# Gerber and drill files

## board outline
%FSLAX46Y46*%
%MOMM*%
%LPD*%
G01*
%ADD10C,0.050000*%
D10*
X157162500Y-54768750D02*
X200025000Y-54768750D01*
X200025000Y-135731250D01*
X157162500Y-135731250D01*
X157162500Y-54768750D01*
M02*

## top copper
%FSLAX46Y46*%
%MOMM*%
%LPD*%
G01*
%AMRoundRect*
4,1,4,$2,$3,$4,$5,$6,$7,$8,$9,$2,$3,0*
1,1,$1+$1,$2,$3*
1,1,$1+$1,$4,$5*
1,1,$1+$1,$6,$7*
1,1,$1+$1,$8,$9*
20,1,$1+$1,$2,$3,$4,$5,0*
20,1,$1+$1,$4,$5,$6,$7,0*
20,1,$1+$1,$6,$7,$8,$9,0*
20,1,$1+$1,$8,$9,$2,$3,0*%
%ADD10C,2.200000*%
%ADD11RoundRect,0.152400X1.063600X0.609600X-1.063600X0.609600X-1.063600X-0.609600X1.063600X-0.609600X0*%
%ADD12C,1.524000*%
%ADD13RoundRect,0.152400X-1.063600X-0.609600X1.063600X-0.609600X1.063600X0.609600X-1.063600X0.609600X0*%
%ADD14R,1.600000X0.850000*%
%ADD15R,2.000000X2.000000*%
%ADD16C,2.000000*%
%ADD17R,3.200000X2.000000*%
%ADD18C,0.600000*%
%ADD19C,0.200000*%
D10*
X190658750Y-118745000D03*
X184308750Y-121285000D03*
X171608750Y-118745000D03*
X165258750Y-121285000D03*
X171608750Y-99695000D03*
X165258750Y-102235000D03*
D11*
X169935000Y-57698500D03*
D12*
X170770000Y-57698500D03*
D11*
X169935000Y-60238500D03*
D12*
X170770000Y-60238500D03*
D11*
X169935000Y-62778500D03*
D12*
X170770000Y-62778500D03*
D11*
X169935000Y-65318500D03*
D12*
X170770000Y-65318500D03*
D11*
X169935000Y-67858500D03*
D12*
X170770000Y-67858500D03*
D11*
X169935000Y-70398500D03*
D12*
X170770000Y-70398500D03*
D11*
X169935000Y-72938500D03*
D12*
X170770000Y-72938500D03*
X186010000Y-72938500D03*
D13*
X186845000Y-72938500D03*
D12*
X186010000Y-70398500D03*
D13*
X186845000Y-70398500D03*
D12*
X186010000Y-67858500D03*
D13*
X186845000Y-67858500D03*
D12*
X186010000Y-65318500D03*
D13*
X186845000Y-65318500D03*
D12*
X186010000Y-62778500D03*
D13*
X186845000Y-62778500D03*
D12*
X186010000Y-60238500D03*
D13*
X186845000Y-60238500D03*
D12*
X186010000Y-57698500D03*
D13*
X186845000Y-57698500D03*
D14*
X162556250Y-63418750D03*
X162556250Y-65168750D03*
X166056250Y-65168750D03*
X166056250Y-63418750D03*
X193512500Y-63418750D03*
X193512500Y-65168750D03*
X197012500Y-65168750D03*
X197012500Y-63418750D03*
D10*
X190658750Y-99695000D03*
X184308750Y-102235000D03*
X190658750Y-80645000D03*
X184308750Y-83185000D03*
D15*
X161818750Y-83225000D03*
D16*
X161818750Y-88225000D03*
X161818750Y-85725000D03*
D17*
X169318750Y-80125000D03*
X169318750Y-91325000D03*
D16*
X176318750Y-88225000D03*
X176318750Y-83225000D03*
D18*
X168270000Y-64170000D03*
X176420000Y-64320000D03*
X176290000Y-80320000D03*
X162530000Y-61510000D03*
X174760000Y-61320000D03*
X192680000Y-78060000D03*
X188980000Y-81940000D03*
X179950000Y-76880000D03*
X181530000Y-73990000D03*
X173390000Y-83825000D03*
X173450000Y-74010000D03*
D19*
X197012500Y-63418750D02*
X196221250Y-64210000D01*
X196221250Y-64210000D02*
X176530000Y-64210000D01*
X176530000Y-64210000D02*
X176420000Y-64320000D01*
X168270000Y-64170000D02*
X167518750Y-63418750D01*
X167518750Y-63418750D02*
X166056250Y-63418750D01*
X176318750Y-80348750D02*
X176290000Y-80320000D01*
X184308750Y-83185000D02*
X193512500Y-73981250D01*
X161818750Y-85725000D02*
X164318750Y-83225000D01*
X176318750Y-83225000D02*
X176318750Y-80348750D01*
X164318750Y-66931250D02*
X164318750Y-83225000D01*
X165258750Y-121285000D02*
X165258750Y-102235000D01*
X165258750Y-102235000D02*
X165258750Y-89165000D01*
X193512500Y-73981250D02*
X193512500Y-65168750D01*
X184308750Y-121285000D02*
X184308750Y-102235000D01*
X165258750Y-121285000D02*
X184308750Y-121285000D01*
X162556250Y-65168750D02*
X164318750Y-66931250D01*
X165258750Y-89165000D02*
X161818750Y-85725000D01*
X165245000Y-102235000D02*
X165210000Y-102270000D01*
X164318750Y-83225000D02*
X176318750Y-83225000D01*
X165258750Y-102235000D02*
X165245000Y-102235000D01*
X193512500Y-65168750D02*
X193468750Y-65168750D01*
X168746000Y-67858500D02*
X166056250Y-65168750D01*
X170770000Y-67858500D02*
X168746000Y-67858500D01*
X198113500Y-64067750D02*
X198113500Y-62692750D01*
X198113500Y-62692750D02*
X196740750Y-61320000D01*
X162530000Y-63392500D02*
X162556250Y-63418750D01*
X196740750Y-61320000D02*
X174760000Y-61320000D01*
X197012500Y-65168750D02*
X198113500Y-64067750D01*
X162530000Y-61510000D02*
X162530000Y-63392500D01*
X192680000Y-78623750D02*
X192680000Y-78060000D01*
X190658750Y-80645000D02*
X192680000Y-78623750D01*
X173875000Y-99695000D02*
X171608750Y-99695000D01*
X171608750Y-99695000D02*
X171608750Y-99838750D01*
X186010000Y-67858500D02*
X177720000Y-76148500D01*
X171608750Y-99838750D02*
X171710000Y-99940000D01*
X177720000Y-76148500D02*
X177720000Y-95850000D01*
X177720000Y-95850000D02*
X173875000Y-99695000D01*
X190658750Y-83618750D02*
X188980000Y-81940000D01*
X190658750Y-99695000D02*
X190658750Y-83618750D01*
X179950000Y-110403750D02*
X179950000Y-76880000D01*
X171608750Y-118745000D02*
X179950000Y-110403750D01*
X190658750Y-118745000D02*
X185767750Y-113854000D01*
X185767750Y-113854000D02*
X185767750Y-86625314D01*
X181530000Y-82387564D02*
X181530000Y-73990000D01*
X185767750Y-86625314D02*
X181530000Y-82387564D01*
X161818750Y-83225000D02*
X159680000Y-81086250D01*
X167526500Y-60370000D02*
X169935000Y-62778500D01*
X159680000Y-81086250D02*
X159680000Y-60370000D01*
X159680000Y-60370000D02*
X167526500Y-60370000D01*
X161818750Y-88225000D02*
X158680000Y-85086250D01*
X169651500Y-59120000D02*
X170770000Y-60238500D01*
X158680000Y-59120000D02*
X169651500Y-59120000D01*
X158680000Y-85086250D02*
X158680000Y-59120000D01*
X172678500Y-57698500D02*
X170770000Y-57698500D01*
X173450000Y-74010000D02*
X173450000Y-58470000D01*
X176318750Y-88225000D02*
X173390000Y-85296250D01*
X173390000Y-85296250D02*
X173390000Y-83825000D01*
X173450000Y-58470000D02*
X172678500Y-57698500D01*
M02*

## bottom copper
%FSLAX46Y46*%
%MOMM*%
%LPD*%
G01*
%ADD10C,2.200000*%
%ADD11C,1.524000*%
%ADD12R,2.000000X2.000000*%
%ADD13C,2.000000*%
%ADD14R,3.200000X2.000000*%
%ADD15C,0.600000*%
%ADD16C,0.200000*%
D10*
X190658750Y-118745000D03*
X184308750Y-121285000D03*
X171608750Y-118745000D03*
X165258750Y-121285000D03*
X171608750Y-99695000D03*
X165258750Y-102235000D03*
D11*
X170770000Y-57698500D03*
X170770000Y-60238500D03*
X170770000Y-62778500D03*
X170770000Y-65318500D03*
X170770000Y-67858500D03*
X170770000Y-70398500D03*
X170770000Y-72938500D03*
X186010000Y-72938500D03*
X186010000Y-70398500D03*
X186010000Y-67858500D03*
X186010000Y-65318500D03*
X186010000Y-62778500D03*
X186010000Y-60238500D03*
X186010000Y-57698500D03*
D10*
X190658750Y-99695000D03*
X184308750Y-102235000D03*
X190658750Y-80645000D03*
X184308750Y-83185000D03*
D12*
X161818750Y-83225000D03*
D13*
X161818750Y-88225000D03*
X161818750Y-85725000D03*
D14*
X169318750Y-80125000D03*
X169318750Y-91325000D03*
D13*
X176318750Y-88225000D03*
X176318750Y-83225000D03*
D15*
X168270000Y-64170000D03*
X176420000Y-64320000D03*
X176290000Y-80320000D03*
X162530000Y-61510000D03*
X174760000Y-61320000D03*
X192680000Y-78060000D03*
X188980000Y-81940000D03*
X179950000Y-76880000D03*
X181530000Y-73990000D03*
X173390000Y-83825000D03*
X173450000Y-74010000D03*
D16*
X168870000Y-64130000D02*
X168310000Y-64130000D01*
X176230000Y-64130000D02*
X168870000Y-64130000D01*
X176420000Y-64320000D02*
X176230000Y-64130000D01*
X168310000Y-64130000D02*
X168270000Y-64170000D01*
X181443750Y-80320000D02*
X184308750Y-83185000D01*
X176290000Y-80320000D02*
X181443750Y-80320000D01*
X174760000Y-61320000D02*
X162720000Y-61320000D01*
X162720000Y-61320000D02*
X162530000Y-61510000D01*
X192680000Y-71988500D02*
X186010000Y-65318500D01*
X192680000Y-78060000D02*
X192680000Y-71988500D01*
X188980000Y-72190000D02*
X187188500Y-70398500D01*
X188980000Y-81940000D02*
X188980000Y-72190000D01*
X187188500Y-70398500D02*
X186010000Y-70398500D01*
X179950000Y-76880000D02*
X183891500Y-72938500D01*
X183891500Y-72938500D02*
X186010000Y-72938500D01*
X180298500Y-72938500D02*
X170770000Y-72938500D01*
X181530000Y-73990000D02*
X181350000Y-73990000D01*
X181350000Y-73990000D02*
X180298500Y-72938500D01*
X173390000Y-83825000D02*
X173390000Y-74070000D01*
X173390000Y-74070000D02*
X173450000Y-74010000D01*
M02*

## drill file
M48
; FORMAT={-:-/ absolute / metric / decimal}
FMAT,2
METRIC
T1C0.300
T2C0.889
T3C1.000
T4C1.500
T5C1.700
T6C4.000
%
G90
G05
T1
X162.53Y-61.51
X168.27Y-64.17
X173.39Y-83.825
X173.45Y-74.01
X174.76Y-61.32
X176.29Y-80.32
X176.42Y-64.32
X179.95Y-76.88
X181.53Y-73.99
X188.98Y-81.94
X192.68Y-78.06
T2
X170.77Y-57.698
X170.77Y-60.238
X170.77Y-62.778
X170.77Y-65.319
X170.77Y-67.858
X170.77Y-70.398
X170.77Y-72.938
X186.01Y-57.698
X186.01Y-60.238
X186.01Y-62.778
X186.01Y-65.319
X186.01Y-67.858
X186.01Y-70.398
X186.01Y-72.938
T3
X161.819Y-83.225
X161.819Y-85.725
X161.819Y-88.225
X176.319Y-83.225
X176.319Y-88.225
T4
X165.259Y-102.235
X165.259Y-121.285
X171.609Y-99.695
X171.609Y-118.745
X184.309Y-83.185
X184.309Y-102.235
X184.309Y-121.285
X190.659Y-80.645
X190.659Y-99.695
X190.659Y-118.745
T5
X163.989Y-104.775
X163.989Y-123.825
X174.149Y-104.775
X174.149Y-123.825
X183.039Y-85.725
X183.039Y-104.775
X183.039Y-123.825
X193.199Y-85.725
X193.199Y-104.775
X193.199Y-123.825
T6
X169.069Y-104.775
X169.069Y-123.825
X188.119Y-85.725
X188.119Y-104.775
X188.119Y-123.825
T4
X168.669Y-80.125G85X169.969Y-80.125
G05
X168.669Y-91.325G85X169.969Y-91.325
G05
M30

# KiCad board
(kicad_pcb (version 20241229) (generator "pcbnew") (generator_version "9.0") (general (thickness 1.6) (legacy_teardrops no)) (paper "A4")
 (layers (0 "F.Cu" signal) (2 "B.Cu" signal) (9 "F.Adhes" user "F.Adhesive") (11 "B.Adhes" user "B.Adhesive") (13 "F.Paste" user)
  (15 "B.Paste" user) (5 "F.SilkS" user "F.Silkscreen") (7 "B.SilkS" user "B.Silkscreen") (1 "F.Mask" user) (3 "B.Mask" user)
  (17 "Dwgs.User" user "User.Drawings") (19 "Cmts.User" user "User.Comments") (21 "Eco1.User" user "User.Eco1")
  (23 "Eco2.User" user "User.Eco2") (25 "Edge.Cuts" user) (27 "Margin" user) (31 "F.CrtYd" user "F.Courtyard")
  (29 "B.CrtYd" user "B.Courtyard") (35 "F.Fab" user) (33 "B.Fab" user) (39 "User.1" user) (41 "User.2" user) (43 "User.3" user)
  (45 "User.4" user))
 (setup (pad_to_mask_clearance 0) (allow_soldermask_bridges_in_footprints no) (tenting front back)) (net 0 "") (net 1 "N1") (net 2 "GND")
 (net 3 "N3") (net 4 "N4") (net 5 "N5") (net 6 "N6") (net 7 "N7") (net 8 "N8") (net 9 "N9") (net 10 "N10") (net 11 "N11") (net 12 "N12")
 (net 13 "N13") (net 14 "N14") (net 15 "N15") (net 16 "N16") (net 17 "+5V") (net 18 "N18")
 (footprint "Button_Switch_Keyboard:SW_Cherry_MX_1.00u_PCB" (layer "F.Cu") (at 190.65875 118.745)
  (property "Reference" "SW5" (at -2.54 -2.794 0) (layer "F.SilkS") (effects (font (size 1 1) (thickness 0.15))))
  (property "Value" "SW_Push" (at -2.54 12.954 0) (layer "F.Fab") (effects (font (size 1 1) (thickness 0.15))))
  (pad "" np_thru_hole circle (at -7.62 5.08) (size 1.7 1.7) (drill 1.7) (layers "*.Cu" "*.Mask"))
  (pad "" np_thru_hole circle (at -2.54 5.08) (size 4 4) (drill 4) (layers "*.Cu" "*.Mask"))
  (pad "" np_thru_hole circle (at 2.54 5.08) (size 1.7 1.7) (drill 1.7) (layers "*.Cu" "*.Mask"))
  (pad "1" thru_hole circle (at 0 0) (size 2.2 2.2) (drill 1.5) (layers "*.Cu" "*.Mask") (remove_unused_layers no) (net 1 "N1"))
  (pad "2" thru_hole circle (at -6.35 2.54) (size 2.2 2.2) (drill 1.5) (layers "*.Cu" "*.Mask") (remove_unused_layers no) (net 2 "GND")))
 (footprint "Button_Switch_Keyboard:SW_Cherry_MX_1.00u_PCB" (layer "F.Cu") (at 171.60875 118.745)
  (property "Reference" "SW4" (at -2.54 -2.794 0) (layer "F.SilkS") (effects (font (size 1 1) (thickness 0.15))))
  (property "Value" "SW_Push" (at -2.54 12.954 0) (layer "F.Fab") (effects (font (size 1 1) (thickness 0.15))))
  (pad "" np_thru_hole circle (at -7.62 5.08) (size 1.7 1.7) (drill 1.7) (layers "*.Cu" "*.Mask"))
  (pad "" np_thru_hole circle (at -2.54 5.08) (size 4 4) (drill 4) (layers "*.Cu" "*.Mask"))
  (pad "" np_thru_hole circle (at 2.54 5.08) (size 1.7 1.7) (drill 1.7) (layers "*.Cu" "*.Mask"))
  (pad "1" thru_hole circle (at 0 0) (size 2.2 2.2) (drill 1.5) (layers "*.Cu" "*.Mask") (remove_unused_layers no) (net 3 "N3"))
  (pad "2" thru_hole circle (at -6.35 2.54) (size 2.2 2.2) (drill 1.5) (layers "*.Cu" "*.Mask") (remove_unused_layers no) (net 2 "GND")))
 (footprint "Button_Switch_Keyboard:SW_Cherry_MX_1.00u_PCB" (layer "F.Cu") (at 171.60875 99.695)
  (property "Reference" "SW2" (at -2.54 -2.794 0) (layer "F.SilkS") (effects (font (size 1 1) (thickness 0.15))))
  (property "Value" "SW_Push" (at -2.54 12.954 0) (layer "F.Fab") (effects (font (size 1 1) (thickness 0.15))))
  (pad "" np_thru_hole circle (at -7.62 5.08) (size 1.7 1.7) (drill 1.7) (layers "*.Cu" "*.Mask"))
  (pad "" np_thru_hole circle (at -2.54 5.08) (size 4 4) (drill 4) (layers "*.Cu" "*.Mask"))
  (pad "" np_thru_hole circle (at 2.54 5.08) (size 1.7 1.7) (drill 1.7) (layers "*.Cu" "*.Mask"))
  (pad "1" thru_hole circle (at 0 0) (size 2.2 2.2) (drill 1.5) (layers "*.Cu" "*.Mask") (remove_unused_layers no) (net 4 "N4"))
  (pad "2" thru_hole circle (at -6.35 2.54) (size 2.2 2.2) (drill 1.5) (layers "*.Cu" "*.Mask") (remove_unused_layers no) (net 2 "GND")))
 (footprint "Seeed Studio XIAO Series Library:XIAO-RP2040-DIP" (layer "F.Cu") (at 178.39 65.3185)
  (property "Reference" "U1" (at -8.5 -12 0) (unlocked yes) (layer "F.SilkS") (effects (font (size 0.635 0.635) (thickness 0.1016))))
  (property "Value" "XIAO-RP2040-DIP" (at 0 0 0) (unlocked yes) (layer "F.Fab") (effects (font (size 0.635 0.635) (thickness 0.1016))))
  (pad "1" smd roundrect (at -8.455 -7.62 180) (size 2.432 1.524) (layers "F.Cu" "F.Mask") (roundrect_rratio 0.1) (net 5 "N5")
   (thermal_bridge_angle 45))
  (pad "1" thru_hole circle (at -7.62 -7.62 180) (size 1.524 1.524) (drill 0.889) (layers "*.Cu" "*.Mask") (remove_unused_layers no)
   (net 5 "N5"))
  (pad "2" smd roundrect (at -8.455 -5.08 180) (size 2.432 1.524) (layers "F.Cu" "F.Mask") (roundrect_rratio 0.1) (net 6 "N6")
   (thermal_bridge_angle 45))
  (pad "2" thru_hole circle (at -7.62 -5.08 180) (size 1.524 1.524) (drill 0.889) (layers "*.Cu" "*.Mask") (remove_unused_layers no)
   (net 6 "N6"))
  (pad "3" smd roundrect (at -8.455 -2.54 180) (size 2.432 1.524) (layers "F.Cu" "F.Mask") (roundrect_rratio 0.1) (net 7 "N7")
   (thermal_bridge_angle 45))
  (pad "3" thru_hole circle (at -7.62 -2.54 180) (size 1.524 1.524) (drill 0.889) (layers "*.Cu" "*.Mask") (remove_unused_layers no)
   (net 7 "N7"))
  (pad "4" smd roundrect (at -8.455 0 180) (size 2.432 1.524) (layers "F.Cu" "F.Mask") (roundrect_rratio 0.1) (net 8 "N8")
   (thermal_bridge_angle 45))
  (pad "4" thru_hole circle (at -7.62 0 180) (size 1.524 1.524) (drill 0.889) (layers "*.Cu" "*.Mask") (remove_unused_layers no)
   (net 8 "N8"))
  (pad "5" smd roundrect (at -8.455 2.54 180) (size 2.432 1.524) (layers "F.Cu" "F.Mask") (roundrect_rratio 0.1) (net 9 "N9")
   (thermal_bridge_angle 45))
  (pad "5" thru_hole circle (at -7.62 2.54 180) (size 1.524 1.524) (drill 0.889) (layers "*.Cu" "*.Mask") (remove_unused_layers no)
   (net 9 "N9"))
  (pad "6" smd roundrect (at -8.455 5.08 180) (size 2.432 1.524) (layers "F.Cu" "F.Mask") (roundrect_rratio 0.1) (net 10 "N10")
   (thermal_bridge_angle 45))
  (pad "6" thru_hole circle (at -7.62 5.08 180) (size 1.524 1.524) (drill 0.889) (layers "*.Cu" "*.Mask") (remove_unused_layers no)
   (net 10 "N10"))
  (pad "7" smd roundrect (at -8.455 7.62 180) (size 2.432 1.524) (layers "F.Cu" "F.Mask") (roundrect_rratio 0.1) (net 1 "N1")
   (thermal_bridge_angle 45))
  (pad "7" thru_hole circle (at -7.62 7.62 180) (size 1.524 1.524) (drill 0.889) (layers "*.Cu" "*.Mask") (remove_unused_layers no)
   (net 1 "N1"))
  (pad "8" thru_hole circle (at 7.62 7.62) (size 1.524 1.524) (drill 0.889) (layers "*.Cu" "*.Mask") (remove_unused_layers no) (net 3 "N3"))
  (pad "8" smd roundrect (at 8.455 7.62) (size 2.432 1.524) (layers "F.Cu" "F.Mask") (roundrect_rratio 0.1) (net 3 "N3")
   (thermal_bridge_angle 45))
  (pad "9" thru_hole circle (at 7.62 5.08) (size 1.524 1.524) (drill 0.889) (layers "*.Cu" "*.Mask") (remove_unused_layers no)
   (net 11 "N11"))
  (pad "9" smd roundrect (at 8.455 5.08) (size 2.432 1.524) (layers "F.Cu" "F.Mask") (roundrect_rratio 0.1) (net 11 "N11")
   (thermal_bridge_angle 45))
  (pad "10" thru_hole circle (at 7.62 2.54) (size 1.524 1.524) (drill 0.889) (layers "*.Cu" "*.Mask") (remove_unused_layers no) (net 4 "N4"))
  (pad "10" smd roundrect (at 8.455 2.54) (size 2.432 1.524) (layers "F.Cu" "F.Mask") (roundrect_rratio 0.1) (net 4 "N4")
   (thermal_bridge_angle 45))
  (pad "11" thru_hole circle (at 7.62 0) (size 1.524 1.524) (drill 0.889) (layers "*.Cu" "*.Mask") (remove_unused_layers no) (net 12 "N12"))
  (pad "11" smd roundrect (at 8.455 0) (size 2.432 1.524) (layers "F.Cu" "F.Mask") (roundrect_rratio 0.1) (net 12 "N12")
   (thermal_bridge_angle 45))
  (pad "12" thru_hole circle (at 7.62 -2.54) (size 1.524 1.524) (drill 0.889) (layers "*.Cu" "*.Mask") (remove_unused_layers no)
   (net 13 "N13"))
  (pad "12" smd roundrect (at 8.455 -2.54) (size 2.432 1.524) (layers "F.Cu" "F.Mask") (roundrect_rratio 0.1) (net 13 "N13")
   (thermal_bridge_angle 45))
  (pad "13" thru_hole circle (at 7.62 -5.08) (size 1.524 1.524) (drill 0.889) (layers "*.Cu" "*.Mask") (remove_unused_layers no)
   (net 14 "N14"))
  (pad "13" smd roundrect (at 8.455 -5.08) (size 2.432 1.524) (layers "F.Cu" "F.Mask") (roundrect_rratio 0.1) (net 14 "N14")
   (thermal_bridge_angle 45))
  (pad "14" thru_hole circle (at 7.62 -7.62) (size 1.524 1.524) (drill 0.889) (layers "*.Cu" "*.Mask") (remove_unused_layers no)
   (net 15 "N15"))
  (pad "14" smd roundrect (at 8.455 -7.62) (size 2.432 1.524) (layers "F.Cu" "F.Mask") (roundrect_rratio 0.1) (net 15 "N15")
   (thermal_bridge_angle 45)))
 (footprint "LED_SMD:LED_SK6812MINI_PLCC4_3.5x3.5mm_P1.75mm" (layer "F.Cu") (at 164.30625 64.29375)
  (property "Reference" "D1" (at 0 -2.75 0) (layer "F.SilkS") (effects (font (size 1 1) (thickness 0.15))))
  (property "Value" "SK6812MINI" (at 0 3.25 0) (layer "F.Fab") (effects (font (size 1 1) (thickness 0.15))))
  (pad "1" smd rect (at -1.75 -0.875) (size 1.6 0.85) (layers "F.Cu" "F.Mask" "F.Paste") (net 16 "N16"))
  (pad "2" smd rect (at -1.75 0.875) (size 1.6 0.85) (layers "F.Cu" "F.Mask" "F.Paste") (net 2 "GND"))
  (pad "3" smd rect (at 1.75 0.875) (size 1.6 0.85) (layers "F.Cu" "F.Mask" "F.Paste") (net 9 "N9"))
  (pad "4" smd rect (at 1.75 -0.875) (size 1.6 0.85) (layers "F.Cu" "F.Mask" "F.Paste") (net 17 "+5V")))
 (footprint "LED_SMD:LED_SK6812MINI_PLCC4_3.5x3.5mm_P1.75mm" (layer "F.Cu") (at 195.2625 64.29375)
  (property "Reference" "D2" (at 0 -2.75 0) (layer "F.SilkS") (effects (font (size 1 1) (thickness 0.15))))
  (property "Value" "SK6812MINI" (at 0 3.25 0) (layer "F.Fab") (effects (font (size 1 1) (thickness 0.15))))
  (pad "1" smd rect (at -1.75 -0.875) (size 1.6 0.85) (layers "F.Cu" "F.Mask" "F.Paste") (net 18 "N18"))
  (pad "2" smd rect (at -1.75 0.875) (size 1.6 0.85) (layers "F.Cu" "F.Mask" "F.Paste") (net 2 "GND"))
  (pad "3" smd rect (at 1.75 0.875) (size 1.6 0.85) (layers "F.Cu" "F.Mask" "F.Paste") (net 16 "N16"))
  (pad "4" smd rect (at 1.75 -0.875) (size 1.6 0.85) (layers "F.Cu" "F.Mask" "F.Paste") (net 17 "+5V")))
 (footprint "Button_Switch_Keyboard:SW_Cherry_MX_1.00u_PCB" (layer "F.Cu") (at 190.65875 99.695)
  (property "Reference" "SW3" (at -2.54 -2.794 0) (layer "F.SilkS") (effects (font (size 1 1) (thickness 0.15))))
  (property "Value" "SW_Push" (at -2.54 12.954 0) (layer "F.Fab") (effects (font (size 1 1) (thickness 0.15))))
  (pad "" np_thru_hole circle (at -7.62 5.08) (size 1.7 1.7) (drill 1.7) (layers "*.Cu" "*.Mask"))
  (pad "" np_thru_hole circle (at -2.54 5.08) (size 4 4) (drill 4) (layers "*.Cu" "*.Mask"))
  (pad "" np_thru_hole circle (at 2.54 5.08) (size 1.7 1.7) (drill 1.7) (layers "*.Cu" "*.Mask"))
  (pad "1" thru_hole circle (at 0 0) (size 2.2 2.2) (drill 1.5) (layers "*.Cu" "*.Mask") (remove_unused_layers no) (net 11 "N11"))
  (pad "2" thru_hole circle (at -6.35 2.54) (size 2.2 2.2) (drill 1.5) (layers "*.Cu" "*.Mask") (remove_unused_layers no) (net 2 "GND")))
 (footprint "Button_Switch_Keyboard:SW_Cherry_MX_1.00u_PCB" (layer "F.Cu") (at 190.65875 80.645)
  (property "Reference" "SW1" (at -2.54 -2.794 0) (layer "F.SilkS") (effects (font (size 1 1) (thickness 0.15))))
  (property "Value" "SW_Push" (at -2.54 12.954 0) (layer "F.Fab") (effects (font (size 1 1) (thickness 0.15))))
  (pad "" np_thru_hole circle (at -7.62 5.08) (size 1.7 1.7) (drill 1.7) (layers "*.Cu" "*.Mask"))
  (pad "" np_thru_hole circle (at -2.54 5.08) (size 4 4) (drill 4) (layers "*.Cu" "*.Mask"))
  (pad "" np_thru_hole circle (at 2.54 5.08) (size 1.7 1.7) (drill 1.7) (layers "*.Cu" "*.Mask"))
  (pad "1" thru_hole circle (at 0 0) (size 2.2 2.2) (drill 1.5) (layers "*.Cu" "*.Mask") (remove_unused_layers no) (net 12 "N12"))
  (pad "2" thru_hole circle (at -6.35 2.54) (size 2.2 2.2) (drill 1.5) (layers "*.Cu" "*.Mask") (remove_unused_layers no) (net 2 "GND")))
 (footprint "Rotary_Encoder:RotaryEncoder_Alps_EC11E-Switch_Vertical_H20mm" (layer "F.Cu") (at 161.81875 83.225)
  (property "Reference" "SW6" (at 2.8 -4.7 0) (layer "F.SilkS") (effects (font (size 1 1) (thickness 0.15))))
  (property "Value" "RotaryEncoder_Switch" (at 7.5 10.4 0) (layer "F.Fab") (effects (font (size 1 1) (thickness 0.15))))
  (pad "A" thru_hole rect (at 0 0) (size 2 2) (drill 1) (layers "*.Cu" "*.Mask") (remove_unused_layers no) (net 7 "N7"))
  (pad "B" thru_hole circle (at 0 5) (size 2 2) (drill 1) (layers "*.Cu" "*.Mask") (remove_unused_layers no) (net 6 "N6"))
  (pad "C" thru_hole circle (at 0 2.5) (size 2 2) (drill 1) (layers "*.Cu" "*.Mask") (remove_unused_layers no) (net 2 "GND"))
  (pad "MP" thru_hole rect (at 7.5 -3.1) (size 3.2 2) (drill oval 2.8 1.5) (layers "*.Cu" "*.Mask") (remove_unused_layers no))
  (pad "MP" thru_hole rect (at 7.5 8.1) (size 3.2 2) (drill oval 2.8 1.5) (layers "*.Cu" "*.Mask") (remove_unused_layers no))
  (pad "S1" thru_hole circle (at 14.5 5) (size 2 2) (drill 1) (layers "*.Cu" "*.Mask") (remove_unused_layers no) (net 5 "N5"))
  (pad "S2" thru_hole circle (at 14.5 0) (size 2 2) (drill 1) (layers "*.Cu" "*.Mask") (remove_unused_layers no) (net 2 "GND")))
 (gr_rect (start 157.1625 54.76875) (end 200.025 135.73125) (stroke (width 0.05) (type default)) (fill no) (layer "Edge.Cuts"))
 (segment (start 197.0125 63.41875) (end 196.22125 64.21) (width 0.2) (layer "F.Cu") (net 17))
 (segment (start 196.22125 64.21) (end 176.53 64.21) (width 0.2) (layer "F.Cu") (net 17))
 (segment (start 176.53 64.21) (end 176.42 64.32) (width 0.2) (layer "F.Cu") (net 17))
 (segment (start 168.27 64.17) (end 167.51875 63.41875) (width 0.2) (layer "F.Cu") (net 17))
 (segment (start 167.51875 63.41875) (end 166.05625 63.41875) (width 0.2) (layer "F.Cu") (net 17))
 (via (at 168.27 64.17) (size 0.6) (drill 0.3) (layers "F.Cu" "B.Cu") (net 17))
 (via (at 176.42 64.32) (size 0.6) (drill 0.3) (layers "F.Cu" "B.Cu") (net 17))
 (segment (start 168.87 64.13) (end 168.31 64.13) (width 0.2) (layer "B.Cu") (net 17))
 (segment (start 176.23 64.13) (end 168.87 64.13) (width 0.2) (layer "B.Cu") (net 17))
 (segment (start 176.42 64.32) (end 176.23 64.13) (width 0.2) (layer "B.Cu") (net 17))
 (segment (start 168.31 64.13) (end 168.27 64.17) (width 0.2) (layer "B.Cu") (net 17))
 (segment (start 176.31875 80.34875) (end 176.29 80.32) (width 0.2) (layer "F.Cu") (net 2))
 (segment (start 184.30875 83.185) (end 193.5125 73.98125) (width 0.2) (layer "F.Cu") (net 2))
 (segment (start 161.81875 85.725) (end 164.31875 83.225) (width 0.2) (layer "F.Cu") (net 2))
 (segment (start 176.31875 83.225) (end 176.31875 80.34875) (width 0.2) (layer "F.Cu") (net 2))
 (segment (start 164.31875 66.93125) (end 164.31875 83.225) (width 0.2) (layer "F.Cu") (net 2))
 (segment (start 165.25875 121.285) (end 165.25875 102.235) (width 0.2) (layer "F.Cu") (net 2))
 (segment (start 165.25875 102.235) (end 165.25875 89.165) (width 0.2) (layer "F.Cu") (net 2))
 (segment (start 193.5125 73.98125) (end 193.5125 65.16875) (width 0.2) (layer "F.Cu") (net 2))
 (segment (start 184.30875 121.285) (end 184.30875 102.235) (width 0.2) (layer "F.Cu") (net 2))
 (segment (start 165.25875 121.285) (end 184.30875 121.285) (width 0.2) (layer "F.Cu") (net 2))
 (segment (start 162.55625 65.16875) (end 164.31875 66.93125) (width 0.2) (layer "F.Cu") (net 2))
 (segment (start 165.25875 89.165) (end 161.81875 85.725) (width 0.2) (layer "F.Cu") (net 2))
 (segment (start 165.245 102.235) (end 165.21 102.27) (width 0.2) (layer "F.Cu") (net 2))
 (segment (start 164.31875 83.225) (end 176.31875 83.225) (width 0.2) (layer "F.Cu") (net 2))
 (segment (start 165.25875 102.235) (end 165.245 102.235) (width 0.2) (layer "F.Cu") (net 2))
 (segment (start 193.5125 65.16875) (end 193.46875 65.16875) (width 0.2) (layer "F.Cu") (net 2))
 (via (at 176.29 80.32) (size 0.6) (drill 0.3) (layers "F.Cu" "B.Cu") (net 2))
 (segment (start 181.44375 80.32) (end 184.30875 83.185) (width 0.2) (layer "B.Cu") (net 2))
 (segment (start 176.29 80.32) (end 181.44375 80.32) (width 0.2) (layer "B.Cu") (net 2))
 (segment (start 168.746 67.8585) (end 166.05625 65.16875) (width 0.2) (layer "F.Cu") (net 9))
 (segment (start 170.77 67.8585) (end 168.746 67.8585) (width 0.2) (layer "F.Cu") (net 9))
 (segment (start 198.1135 64.06775) (end 198.1135 62.69275) (width 0.2) (layer "F.Cu") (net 16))
 (segment (start 198.1135 62.69275) (end 196.74075 61.32) (width 0.2) (layer "F.Cu") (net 16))
 (segment (start 162.53 63.3925) (end 162.55625 63.41875) (width 0.2) (layer "F.Cu") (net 16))
 (segment (start 196.74075 61.32) (end 174.76 61.32) (width 0.2) (layer "F.Cu") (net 16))
 (segment (start 197.0125 65.16875) (end 198.1135 64.06775) (width 0.2) (layer "F.Cu") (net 16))
 (segment (start 162.53 61.51) (end 162.53 63.3925) (width 0.2) (layer "F.Cu") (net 16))
 (via (at 162.53 61.51) (size 0.6) (drill 0.3) (layers "F.Cu" "B.Cu") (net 16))
 (via (at 174.76 61.32) (size 0.6) (drill 0.3) (layers "F.Cu" "B.Cu") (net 16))
 (segment (start 174.76 61.32) (end 162.72 61.32) (width 0.2) (layer "B.Cu") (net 16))
 (segment (start 162.72 61.32) (end 162.53 61.51) (width 0.2) (layer "B.Cu") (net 16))
 (segment (start 192.68 78.62375) (end 192.68 78.06) (width 0.2) (layer "F.Cu") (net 12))
 (segment (start 190.65875 80.645) (end 192.68 78.62375) (width 0.2) (layer "F.Cu") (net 12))
 (via (at 192.68 78.06) (size 0.6) (drill 0.3) (layers "F.Cu" "B.Cu") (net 12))
 (segment (start 192.68 71.9885) (end 186.01 65.3185) (width 0.2) (layer "B.Cu") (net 12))
 (segment (start 192.68 78.06) (end 192.68 71.9885) (width 0.2) (layer "B.Cu") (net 12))
 (segment (start 173.875 99.695) (end 171.60875 99.695) (width 0.2) (layer "F.Cu") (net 4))
 (segment (start 171.60875 99.695) (end 171.60875 99.83875) (width 0.2) (layer "F.Cu") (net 4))
 (segment (start 186.01 67.8585) (end 177.72 76.1485) (width 0.2) (layer "F.Cu") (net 4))
 (segment (start 171.60875 99.83875) (end 171.71 99.94) (width 0.2) (layer "F.Cu") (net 4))
 (segment (start 177.72 76.1485) (end 177.72 95.85) (width 0.2) (layer "F.Cu") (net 4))
 (segment (start 177.72 95.85) (end 173.875 99.695) (width 0.2) (layer "F.Cu") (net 4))
 (segment (start 190.65875 83.61875) (end 188.98 81.94) (width 0.2) (layer "F.Cu") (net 11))
 (segment (start 190.65875 99.695) (end 190.65875 83.61875) (width 0.2) (layer "F.Cu") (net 11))
 (via (at 188.98 81.94) (size 0.6) (drill 0.3) (layers "F.Cu" "B.Cu") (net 11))
 (segment (start 188.98 72.19) (end 187.1885 70.3985) (width 0.2) (layer "B.Cu") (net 11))
 (segment (start 188.98 81.94) (end 188.98 72.19) (width 0.2) (layer "B.Cu") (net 11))
 (segment (start 187.1885 70.3985) (end 186.01 70.3985) (width 0.2) (layer "B.Cu") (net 11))
 (segment (start 179.95 110.40375) (end 179.95 76.88) (width 0.2) (layer "F.Cu") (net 3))
 (segment (start 171.60875 118.745) (end 179.95 110.40375) (width 0.2) (layer "F.Cu") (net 3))
 (via (at 179.95 76.88) (size 0.6) (drill 0.3) (layers "F.Cu" "B.Cu") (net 3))
 (segment (start 179.95 76.88) (end 183.8915 72.9385) (width 0.2) (layer "B.Cu") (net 3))
 (segment (start 183.8915 72.9385) (end 186.01 72.9385) (width 0.2) (layer "B.Cu") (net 3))
 (segment (start 190.65875 118.745) (end 185.76775 113.854) (width 0.2) (layer "F.Cu") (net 1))
 (segment (start 185.76775 113.854) (end 185.76775 86.625314) (width 0.2) (layer "F.Cu") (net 1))
 (segment (start 181.53 82.387564) (end 181.53 73.99) (width 0.2) (layer "F.Cu") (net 1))
 (segment (start 185.76775 86.625314) (end 181.53 82.387564) (width 0.2) (layer "F.Cu") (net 1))
 (via (at 181.53 73.99) (size 0.6) (drill 0.3) (layers "F.Cu" "B.Cu") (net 1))
 (segment (start 180.2985 72.9385) (end 170.77 72.9385) (width 0.2) (layer "B.Cu") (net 1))
 (segment (start 181.53 73.99) (end 181.35 73.99) (width 0.2) (layer "B.Cu") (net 1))
 (segment (start 181.35 73.99) (end 180.2985 72.9385) (width 0.2) (layer "B.Cu") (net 1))
 (segment (start 161.81875 83.225) (end 159.68 81.08625) (width 0.2) (layer "F.Cu") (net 7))
 (segment (start 167.5265 60.37) (end 169.935 62.7785) (width 0.2) (layer "F.Cu") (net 7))
 (segment (start 159.68 81.08625) (end 159.68 60.37) (width 0.2) (layer "F.Cu") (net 7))
 (segment (start 159.68 60.37) (end 167.5265 60.37) (width 0.2) (layer "F.Cu") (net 7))
 (segment (start 161.81875 88.225) (end 158.68 85.08625) (width 0.2) (layer "F.Cu") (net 6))
 (segment (start 169.6515 59.12) (end 170.77 60.2385) (width 0.2) (layer "F.Cu") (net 6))
 (segment (start 158.68 59.12) (end 169.6515 59.12) (width 0.2) (layer "F.Cu") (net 6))
 (segment (start 158.68 85.08625) (end 158.68 59.12) (width 0.2) (layer "F.Cu") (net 6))
 (segment (start 172.6785 57.6985) (end 170.77 57.6985) (width 0.2) (layer "F.Cu") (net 5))
 (segment (start 173.45 74.01) (end 173.45 58.47) (width 0.2) (layer "F.Cu") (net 5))
 (segment (start 176.31875 88.225) (end 173.39 85.29625) (width 0.2) (layer "F.Cu") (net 5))
 (segment (start 173.39 85.29625) (end 173.39 83.825) (width 0.2) (layer "F.Cu") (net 5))
 (segment (start 173.45 58.47) (end 172.6785 57.6985) (width 0.2) (layer "F.Cu") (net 5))
 (via (at 173.39 83.825) (size 0.6) (drill 0.3) (layers "F.Cu" "B.Cu") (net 5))
 (via (at 173.45 74.01) (size 0.6) (drill 0.3) (layers "F.Cu" "B.Cu") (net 5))
 (segment (start 173.39 83.825) (end 173.39 74.07) (width 0.2) (layer "B.Cu") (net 5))
 (segment (start 173.39 74.07) (end 173.45 74.01) (width 0.2) (layer "B.Cu") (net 5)))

